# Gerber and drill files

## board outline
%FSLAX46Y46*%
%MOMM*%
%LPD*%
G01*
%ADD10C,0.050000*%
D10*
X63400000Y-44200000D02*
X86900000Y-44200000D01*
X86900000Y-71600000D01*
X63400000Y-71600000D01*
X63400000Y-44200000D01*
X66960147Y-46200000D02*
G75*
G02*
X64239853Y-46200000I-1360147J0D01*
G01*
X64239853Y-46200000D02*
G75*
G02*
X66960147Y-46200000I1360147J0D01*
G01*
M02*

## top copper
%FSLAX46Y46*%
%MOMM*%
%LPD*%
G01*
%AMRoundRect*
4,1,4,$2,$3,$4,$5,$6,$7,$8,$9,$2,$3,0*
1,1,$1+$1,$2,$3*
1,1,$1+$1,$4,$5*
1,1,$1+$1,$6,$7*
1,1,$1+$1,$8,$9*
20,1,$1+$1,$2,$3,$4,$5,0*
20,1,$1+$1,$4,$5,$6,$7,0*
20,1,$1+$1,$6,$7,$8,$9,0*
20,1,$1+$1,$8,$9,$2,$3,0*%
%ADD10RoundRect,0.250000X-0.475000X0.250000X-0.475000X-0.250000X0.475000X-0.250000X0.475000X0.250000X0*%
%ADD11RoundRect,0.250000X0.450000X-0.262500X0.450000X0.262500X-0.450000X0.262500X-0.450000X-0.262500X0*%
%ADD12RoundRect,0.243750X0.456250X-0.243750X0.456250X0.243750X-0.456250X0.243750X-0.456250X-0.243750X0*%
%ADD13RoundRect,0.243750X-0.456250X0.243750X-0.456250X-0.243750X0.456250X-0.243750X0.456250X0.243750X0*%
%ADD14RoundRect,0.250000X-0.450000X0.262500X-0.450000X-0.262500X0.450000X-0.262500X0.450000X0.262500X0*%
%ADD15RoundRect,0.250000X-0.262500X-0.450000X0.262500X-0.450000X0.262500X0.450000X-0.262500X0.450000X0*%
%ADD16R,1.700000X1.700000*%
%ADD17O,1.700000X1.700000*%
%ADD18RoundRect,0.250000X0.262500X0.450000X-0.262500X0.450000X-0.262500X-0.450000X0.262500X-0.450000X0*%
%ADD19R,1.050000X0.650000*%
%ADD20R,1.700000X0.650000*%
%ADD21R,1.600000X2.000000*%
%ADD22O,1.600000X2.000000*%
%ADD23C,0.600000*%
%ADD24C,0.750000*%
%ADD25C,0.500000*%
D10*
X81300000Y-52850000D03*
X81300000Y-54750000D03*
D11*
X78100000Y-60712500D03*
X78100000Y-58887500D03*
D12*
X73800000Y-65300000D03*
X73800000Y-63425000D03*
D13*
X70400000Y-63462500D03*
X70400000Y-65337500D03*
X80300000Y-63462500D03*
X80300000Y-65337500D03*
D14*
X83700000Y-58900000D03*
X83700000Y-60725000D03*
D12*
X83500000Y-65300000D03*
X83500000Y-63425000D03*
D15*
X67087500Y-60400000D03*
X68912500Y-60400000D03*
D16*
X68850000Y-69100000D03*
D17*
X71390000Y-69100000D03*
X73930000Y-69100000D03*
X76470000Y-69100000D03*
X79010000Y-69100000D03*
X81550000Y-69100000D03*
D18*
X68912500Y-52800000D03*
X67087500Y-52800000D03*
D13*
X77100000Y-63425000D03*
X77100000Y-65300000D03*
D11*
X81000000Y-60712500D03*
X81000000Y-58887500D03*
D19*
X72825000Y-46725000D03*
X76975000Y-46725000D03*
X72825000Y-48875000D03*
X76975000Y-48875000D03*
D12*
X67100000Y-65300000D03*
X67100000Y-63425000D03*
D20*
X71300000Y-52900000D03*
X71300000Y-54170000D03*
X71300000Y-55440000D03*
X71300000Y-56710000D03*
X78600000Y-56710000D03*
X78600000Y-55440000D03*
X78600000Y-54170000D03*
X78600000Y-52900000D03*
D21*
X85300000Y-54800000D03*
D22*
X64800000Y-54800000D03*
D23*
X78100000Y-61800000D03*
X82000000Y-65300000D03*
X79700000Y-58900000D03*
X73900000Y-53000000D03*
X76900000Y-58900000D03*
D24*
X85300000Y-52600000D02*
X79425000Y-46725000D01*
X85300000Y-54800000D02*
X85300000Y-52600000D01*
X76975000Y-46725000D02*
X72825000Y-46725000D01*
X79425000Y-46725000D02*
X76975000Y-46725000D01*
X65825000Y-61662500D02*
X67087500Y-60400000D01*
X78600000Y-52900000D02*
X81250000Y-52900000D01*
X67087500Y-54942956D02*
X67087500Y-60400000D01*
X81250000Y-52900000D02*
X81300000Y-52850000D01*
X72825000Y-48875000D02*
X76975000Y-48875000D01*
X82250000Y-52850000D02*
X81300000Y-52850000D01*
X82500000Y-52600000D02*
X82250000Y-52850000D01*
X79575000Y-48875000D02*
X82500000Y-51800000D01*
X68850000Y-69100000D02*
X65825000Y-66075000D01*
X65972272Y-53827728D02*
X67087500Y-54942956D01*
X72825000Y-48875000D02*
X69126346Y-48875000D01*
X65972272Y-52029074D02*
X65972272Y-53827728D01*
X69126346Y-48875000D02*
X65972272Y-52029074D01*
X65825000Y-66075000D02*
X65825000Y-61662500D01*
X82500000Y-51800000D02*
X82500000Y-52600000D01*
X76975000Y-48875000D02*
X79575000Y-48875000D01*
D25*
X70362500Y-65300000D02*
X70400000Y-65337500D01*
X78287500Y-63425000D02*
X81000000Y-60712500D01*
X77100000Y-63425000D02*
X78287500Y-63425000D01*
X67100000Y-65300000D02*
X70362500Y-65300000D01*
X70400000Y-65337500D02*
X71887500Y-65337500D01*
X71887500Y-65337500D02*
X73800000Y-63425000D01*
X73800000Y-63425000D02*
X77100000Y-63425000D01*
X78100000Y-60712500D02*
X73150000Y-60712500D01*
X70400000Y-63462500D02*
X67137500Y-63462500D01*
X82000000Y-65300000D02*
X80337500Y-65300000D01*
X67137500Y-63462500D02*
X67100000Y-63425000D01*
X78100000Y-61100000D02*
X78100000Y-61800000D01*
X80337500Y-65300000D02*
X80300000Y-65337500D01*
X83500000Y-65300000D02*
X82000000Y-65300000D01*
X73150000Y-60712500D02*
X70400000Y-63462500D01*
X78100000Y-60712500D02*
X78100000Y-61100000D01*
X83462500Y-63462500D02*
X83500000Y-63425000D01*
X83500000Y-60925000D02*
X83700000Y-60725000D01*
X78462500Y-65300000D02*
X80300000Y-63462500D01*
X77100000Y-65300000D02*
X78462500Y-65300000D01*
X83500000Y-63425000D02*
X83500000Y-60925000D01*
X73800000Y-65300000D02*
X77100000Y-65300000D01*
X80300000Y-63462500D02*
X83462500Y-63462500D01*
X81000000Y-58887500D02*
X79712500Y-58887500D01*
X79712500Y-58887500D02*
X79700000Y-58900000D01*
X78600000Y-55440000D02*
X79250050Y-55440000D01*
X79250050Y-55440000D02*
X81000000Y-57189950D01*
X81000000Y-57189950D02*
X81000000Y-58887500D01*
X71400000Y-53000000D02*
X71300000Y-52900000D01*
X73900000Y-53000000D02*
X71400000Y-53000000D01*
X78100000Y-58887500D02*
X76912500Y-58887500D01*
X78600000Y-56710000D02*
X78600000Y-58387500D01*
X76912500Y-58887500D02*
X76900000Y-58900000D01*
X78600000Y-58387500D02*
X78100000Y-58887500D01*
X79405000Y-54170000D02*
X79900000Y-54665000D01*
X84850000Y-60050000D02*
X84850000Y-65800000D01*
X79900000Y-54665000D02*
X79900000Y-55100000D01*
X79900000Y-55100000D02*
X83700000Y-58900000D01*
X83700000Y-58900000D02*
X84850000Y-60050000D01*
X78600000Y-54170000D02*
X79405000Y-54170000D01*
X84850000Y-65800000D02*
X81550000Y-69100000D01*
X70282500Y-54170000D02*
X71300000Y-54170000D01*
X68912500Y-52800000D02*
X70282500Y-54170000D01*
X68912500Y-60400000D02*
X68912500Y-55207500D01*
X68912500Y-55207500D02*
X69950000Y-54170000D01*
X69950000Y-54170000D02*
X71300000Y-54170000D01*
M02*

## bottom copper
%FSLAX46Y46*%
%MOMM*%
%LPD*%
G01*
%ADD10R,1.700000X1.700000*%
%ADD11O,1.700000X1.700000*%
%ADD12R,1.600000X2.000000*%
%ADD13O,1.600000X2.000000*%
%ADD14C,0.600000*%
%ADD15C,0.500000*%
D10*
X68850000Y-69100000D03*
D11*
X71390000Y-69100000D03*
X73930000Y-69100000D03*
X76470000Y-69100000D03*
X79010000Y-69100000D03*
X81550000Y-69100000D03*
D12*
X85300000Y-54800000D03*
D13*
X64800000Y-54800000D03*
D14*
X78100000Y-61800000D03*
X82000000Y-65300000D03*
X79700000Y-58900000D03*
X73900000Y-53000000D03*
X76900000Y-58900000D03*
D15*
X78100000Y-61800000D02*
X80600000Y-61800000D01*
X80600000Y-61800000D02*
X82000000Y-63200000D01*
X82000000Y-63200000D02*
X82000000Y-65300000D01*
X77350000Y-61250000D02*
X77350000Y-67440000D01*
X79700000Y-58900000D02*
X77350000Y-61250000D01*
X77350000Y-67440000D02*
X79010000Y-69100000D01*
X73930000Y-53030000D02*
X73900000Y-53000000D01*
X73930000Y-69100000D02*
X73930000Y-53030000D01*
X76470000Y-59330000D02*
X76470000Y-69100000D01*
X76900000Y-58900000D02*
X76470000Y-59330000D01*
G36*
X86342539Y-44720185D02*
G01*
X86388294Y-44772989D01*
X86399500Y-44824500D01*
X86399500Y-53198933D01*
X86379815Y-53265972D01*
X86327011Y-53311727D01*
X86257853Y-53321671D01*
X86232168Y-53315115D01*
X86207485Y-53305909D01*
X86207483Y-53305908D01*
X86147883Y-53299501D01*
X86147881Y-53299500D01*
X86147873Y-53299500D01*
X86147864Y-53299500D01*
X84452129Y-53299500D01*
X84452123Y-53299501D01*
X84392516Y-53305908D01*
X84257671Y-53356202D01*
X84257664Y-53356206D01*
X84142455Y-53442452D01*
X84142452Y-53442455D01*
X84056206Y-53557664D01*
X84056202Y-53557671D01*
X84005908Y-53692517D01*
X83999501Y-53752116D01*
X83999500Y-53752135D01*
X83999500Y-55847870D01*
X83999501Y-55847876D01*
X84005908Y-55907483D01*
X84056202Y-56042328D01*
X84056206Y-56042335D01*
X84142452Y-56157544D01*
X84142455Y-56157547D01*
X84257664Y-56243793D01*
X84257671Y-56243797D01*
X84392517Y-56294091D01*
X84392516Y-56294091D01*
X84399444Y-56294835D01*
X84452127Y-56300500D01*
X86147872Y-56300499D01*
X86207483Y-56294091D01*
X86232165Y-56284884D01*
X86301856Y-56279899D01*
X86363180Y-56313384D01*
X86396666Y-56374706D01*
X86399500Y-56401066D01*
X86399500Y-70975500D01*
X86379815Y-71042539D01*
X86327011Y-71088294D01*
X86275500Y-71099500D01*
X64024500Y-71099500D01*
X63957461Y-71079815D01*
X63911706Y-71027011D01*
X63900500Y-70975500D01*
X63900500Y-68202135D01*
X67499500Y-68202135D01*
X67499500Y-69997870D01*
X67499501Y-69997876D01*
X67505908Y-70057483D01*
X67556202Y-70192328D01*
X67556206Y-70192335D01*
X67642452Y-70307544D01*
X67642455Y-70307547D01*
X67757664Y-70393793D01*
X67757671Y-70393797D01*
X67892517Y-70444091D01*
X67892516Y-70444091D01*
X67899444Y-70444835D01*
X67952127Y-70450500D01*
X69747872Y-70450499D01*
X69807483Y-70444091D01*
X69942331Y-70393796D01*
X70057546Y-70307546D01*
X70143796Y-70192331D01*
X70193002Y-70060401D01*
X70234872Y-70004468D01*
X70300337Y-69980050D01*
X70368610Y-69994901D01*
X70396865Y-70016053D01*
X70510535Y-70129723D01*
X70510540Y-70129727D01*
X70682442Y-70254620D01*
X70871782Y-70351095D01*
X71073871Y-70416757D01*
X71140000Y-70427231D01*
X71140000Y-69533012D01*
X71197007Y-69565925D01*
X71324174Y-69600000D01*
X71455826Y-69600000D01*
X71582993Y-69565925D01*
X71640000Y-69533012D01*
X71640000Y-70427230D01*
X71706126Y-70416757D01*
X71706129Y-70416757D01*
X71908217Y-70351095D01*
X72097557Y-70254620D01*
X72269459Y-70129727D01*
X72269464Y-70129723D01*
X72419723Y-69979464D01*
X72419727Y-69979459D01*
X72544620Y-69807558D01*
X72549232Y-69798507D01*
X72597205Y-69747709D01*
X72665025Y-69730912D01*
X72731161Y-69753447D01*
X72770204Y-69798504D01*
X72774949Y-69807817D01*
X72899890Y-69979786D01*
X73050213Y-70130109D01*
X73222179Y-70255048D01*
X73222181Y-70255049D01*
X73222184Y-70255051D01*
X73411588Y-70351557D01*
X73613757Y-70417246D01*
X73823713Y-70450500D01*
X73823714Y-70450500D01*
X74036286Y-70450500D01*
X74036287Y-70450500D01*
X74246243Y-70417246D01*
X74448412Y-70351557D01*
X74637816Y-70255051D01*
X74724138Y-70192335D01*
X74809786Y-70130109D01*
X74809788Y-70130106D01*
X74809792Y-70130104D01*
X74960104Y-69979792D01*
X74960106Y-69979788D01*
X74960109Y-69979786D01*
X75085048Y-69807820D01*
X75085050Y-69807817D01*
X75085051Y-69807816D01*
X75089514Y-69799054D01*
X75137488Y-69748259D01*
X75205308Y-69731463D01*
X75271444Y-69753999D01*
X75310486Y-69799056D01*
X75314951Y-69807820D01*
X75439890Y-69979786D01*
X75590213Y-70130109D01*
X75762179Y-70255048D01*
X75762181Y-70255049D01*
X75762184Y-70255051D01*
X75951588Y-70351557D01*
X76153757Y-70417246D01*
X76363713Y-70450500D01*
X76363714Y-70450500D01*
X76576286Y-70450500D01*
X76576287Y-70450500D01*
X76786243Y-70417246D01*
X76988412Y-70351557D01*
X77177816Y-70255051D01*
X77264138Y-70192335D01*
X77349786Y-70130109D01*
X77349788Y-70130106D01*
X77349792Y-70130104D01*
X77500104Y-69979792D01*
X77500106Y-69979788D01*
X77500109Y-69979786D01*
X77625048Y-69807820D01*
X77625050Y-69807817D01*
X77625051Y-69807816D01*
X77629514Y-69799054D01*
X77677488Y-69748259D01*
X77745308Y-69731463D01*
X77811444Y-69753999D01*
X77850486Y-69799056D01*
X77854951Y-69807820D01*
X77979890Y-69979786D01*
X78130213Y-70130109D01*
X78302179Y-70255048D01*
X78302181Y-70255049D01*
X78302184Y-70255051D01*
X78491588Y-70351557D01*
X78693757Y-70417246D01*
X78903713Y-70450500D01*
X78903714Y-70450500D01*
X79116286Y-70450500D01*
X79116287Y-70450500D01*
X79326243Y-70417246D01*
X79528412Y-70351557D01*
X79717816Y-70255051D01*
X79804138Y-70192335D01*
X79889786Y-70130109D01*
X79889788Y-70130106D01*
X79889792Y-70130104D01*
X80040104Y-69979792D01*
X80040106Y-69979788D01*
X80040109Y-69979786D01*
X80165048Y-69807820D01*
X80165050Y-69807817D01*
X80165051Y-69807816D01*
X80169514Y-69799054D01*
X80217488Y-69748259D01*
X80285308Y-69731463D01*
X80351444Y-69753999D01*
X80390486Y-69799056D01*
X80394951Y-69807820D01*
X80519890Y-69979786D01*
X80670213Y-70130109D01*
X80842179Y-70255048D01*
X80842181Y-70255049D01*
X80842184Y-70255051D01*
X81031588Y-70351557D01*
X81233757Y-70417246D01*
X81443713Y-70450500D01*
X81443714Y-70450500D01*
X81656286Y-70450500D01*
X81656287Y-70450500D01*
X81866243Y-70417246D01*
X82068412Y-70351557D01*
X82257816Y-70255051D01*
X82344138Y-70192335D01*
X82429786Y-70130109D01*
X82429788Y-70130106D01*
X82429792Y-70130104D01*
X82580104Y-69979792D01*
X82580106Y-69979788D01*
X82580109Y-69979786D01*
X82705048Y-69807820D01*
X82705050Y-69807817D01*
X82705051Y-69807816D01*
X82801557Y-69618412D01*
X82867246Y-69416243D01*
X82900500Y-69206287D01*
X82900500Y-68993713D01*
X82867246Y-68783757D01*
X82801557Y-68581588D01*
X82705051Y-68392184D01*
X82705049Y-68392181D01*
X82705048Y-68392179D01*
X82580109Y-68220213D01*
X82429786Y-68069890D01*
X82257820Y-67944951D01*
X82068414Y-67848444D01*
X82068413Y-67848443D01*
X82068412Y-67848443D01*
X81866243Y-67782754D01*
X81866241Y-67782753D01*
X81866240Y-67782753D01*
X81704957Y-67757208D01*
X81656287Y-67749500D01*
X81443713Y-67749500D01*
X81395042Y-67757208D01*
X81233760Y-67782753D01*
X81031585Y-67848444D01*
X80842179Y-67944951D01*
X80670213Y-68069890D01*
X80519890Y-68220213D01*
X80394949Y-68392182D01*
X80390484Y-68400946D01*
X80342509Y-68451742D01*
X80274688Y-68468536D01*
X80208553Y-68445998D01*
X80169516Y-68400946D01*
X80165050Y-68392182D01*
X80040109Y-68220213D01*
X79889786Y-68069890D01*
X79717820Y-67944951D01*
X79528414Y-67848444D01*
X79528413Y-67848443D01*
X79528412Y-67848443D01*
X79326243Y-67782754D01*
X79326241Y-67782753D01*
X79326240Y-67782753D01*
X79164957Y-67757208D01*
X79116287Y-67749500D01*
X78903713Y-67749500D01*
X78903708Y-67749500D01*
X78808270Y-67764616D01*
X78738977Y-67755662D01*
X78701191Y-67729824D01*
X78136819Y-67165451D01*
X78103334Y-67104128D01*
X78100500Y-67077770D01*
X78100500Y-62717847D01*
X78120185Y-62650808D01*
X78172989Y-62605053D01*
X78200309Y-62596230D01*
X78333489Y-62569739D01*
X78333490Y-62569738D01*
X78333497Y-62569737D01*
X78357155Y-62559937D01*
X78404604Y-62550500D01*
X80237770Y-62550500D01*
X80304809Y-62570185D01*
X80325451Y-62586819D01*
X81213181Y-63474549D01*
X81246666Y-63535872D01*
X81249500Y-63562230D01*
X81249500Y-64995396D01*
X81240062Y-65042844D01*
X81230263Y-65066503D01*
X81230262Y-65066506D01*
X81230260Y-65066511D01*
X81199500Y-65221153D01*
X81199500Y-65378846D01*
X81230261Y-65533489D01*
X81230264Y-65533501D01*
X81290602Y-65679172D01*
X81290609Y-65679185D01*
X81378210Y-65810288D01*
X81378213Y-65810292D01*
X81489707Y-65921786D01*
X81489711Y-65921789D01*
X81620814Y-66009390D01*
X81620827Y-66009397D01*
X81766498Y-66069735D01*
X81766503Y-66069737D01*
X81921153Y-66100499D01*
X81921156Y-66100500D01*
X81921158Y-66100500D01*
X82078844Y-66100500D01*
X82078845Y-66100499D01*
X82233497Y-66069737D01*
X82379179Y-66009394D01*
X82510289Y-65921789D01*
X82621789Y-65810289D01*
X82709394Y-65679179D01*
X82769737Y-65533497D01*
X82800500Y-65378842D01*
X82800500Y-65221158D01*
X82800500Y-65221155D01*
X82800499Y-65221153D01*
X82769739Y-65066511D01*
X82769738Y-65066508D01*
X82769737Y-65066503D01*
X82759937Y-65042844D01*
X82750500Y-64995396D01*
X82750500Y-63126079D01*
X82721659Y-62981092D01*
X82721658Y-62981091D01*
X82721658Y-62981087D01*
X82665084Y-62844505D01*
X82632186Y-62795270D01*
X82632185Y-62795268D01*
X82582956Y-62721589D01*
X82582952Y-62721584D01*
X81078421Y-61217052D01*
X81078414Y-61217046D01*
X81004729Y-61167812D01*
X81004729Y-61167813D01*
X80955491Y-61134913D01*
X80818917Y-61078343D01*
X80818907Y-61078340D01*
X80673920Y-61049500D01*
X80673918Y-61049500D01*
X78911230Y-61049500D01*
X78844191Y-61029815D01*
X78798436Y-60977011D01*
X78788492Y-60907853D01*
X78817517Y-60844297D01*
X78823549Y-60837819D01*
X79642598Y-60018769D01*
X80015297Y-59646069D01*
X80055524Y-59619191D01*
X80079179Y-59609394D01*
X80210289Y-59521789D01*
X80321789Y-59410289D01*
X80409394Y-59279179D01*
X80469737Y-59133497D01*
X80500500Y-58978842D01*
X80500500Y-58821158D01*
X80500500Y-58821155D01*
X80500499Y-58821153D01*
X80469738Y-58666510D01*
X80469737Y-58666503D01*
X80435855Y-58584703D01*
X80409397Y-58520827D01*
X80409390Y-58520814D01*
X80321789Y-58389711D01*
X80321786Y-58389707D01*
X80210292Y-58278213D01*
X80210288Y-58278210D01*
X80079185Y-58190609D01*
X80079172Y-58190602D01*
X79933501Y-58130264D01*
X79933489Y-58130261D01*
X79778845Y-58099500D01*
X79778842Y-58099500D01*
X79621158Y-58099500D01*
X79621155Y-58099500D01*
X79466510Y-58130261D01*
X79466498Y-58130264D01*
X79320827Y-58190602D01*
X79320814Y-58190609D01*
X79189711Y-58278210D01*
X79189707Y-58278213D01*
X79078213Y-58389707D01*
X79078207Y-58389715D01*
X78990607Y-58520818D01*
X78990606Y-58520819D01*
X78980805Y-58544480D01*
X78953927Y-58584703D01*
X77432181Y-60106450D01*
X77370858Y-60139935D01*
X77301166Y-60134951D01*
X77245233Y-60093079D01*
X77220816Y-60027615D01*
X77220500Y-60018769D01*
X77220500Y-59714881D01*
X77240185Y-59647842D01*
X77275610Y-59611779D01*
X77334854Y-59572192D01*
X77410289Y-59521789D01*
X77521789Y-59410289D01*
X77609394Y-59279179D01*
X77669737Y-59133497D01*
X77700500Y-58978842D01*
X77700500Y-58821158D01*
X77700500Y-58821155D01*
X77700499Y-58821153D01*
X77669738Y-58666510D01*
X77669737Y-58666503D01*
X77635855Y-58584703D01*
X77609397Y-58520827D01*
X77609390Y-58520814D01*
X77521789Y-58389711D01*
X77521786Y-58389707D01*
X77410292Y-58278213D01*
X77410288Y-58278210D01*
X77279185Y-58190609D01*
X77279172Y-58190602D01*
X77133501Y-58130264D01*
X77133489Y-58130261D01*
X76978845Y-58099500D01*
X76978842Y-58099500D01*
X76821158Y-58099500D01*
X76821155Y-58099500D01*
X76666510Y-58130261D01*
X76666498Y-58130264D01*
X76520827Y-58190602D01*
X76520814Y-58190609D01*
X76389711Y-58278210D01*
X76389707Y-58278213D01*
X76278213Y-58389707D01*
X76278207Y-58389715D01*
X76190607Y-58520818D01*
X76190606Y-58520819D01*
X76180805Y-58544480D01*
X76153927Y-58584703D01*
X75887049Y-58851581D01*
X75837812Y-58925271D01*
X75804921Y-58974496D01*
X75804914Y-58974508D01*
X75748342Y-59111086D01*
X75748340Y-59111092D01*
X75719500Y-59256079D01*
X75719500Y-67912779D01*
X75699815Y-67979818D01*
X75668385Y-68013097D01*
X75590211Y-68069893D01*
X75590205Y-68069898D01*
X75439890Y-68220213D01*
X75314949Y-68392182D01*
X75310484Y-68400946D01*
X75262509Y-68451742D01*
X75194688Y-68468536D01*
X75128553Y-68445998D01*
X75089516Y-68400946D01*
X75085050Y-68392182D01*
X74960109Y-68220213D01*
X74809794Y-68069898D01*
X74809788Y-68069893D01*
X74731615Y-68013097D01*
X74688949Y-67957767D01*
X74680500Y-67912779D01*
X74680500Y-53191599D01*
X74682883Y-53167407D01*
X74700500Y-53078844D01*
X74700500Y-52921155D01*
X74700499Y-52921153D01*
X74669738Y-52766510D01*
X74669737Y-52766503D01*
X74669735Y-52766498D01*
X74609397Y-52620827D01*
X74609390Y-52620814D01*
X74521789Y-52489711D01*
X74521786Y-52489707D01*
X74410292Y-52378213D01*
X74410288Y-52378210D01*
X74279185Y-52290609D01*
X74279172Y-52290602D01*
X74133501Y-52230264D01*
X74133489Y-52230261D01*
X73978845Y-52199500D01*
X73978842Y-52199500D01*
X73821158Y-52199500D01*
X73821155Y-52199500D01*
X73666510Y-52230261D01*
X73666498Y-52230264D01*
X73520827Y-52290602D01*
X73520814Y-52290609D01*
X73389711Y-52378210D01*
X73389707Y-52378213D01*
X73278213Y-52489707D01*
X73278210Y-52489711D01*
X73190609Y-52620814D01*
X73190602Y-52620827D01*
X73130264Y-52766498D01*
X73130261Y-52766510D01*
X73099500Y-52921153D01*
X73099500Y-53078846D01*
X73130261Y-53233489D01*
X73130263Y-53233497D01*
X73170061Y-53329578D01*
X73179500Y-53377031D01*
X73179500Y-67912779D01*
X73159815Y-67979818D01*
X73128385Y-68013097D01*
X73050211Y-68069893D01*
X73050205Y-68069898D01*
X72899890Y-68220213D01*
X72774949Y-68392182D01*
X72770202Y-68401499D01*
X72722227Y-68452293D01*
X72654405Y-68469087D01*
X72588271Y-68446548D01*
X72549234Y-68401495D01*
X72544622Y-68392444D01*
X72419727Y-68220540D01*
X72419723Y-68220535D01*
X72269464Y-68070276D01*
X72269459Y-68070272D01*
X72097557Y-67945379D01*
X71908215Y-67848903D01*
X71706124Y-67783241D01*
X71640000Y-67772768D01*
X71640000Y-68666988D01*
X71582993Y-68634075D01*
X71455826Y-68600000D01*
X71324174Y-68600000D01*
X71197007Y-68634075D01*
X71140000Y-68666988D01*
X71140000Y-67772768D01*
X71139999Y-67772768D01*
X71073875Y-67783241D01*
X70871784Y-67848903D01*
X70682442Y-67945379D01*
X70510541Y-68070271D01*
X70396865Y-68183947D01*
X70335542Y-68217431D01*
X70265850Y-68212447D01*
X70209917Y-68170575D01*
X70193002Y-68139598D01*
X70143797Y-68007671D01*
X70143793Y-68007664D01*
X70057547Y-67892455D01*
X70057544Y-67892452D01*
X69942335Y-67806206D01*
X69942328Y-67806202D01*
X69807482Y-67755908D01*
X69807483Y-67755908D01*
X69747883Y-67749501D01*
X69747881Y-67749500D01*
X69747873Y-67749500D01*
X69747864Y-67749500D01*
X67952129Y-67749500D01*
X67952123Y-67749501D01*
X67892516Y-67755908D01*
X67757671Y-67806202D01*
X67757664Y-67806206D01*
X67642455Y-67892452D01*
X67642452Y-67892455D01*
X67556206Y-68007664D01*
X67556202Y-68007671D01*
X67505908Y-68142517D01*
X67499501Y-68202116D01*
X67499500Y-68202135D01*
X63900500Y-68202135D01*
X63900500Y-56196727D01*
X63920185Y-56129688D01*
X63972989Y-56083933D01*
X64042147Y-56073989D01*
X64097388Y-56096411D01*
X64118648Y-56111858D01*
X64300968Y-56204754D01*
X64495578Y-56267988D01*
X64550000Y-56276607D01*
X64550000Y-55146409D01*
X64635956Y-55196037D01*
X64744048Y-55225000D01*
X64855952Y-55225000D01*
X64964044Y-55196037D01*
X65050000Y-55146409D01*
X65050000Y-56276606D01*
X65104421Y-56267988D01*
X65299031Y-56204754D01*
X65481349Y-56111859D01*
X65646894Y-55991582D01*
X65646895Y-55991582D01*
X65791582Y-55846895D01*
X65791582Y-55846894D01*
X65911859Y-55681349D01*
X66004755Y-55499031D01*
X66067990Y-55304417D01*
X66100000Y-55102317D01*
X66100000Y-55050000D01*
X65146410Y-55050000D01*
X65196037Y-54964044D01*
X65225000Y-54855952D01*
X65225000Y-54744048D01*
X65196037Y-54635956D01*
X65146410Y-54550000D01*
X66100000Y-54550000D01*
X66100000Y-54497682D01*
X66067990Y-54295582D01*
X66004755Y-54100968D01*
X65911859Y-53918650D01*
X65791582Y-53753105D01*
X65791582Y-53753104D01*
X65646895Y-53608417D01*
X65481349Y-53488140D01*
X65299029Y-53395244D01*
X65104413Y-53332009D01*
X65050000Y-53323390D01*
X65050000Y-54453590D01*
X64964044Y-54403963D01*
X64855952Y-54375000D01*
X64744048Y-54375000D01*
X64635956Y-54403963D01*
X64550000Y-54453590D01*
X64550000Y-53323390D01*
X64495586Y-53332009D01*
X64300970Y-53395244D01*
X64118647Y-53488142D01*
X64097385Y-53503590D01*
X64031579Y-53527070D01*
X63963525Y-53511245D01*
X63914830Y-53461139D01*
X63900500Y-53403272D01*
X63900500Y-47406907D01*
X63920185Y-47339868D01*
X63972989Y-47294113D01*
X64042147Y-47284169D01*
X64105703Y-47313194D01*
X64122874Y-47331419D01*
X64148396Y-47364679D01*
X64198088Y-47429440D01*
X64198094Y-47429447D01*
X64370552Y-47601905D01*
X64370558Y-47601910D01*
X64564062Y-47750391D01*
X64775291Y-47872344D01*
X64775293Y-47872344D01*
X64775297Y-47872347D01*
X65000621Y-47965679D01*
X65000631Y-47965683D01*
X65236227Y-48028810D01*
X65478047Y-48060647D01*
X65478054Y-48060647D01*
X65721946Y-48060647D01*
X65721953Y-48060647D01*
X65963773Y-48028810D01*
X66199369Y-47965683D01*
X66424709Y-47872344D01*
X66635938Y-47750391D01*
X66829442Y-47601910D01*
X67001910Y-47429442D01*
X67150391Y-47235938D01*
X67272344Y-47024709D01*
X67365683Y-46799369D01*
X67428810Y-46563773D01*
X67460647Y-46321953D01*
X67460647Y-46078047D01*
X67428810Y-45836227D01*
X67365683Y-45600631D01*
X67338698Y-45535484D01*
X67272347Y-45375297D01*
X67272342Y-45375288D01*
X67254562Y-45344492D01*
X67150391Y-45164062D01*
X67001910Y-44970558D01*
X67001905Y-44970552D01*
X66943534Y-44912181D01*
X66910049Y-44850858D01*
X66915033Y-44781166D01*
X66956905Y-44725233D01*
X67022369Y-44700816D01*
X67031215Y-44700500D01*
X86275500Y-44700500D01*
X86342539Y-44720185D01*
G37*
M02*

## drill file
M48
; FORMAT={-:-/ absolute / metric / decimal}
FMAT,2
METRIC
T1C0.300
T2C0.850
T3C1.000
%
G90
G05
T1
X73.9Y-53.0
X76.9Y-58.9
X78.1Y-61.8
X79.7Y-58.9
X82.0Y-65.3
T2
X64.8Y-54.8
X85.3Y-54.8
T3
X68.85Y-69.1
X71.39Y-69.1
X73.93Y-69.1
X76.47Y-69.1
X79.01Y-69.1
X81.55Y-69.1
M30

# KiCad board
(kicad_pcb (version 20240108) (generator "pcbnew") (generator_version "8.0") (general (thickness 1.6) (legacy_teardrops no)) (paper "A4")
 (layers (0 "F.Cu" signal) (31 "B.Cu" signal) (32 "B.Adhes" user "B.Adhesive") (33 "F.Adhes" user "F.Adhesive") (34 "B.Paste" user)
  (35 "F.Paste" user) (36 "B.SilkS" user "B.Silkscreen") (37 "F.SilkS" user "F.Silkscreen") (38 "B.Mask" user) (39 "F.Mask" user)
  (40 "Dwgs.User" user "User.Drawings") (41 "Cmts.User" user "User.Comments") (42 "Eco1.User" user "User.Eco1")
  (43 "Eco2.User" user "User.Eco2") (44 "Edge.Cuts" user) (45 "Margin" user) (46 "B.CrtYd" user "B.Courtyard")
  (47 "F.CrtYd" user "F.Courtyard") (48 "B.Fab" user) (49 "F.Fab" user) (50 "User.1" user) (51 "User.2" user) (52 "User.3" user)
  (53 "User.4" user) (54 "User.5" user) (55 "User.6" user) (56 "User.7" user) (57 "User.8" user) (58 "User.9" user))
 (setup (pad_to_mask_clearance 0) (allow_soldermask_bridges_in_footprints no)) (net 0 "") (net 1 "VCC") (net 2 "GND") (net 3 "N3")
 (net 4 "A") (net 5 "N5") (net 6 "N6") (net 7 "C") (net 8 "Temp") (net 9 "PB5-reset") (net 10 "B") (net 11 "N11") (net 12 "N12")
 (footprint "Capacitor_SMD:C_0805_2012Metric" (layer "F.Cu") (at 81.3 53.8 -90)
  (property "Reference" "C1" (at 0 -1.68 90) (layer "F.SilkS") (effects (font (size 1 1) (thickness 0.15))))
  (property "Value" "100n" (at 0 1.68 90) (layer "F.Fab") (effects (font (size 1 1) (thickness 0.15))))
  (pad "1" smd roundrect (at -0.95 0 270) (size 1 1.45) (layers "F.Cu" "F.Paste" "F.Mask") (roundrect_rratio 0.25) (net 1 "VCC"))
  (pad "2" smd roundrect (at 0.95 0 270) (size 1 1.45) (layers "F.Cu" "F.Paste" "F.Mask") (roundrect_rratio 0.25) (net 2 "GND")))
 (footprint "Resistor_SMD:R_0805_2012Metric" (layer "F.Cu") (at 78.1 59.8 90)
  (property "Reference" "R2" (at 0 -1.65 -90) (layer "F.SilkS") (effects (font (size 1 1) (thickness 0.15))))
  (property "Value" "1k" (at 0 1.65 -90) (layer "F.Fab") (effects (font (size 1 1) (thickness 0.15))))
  (pad "1" smd roundrect (at -0.9125 0 90) (size 1.025 1.4) (layers "F.Cu" "F.Paste" "F.Mask") (roundrect_rratio 0.243902) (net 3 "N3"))
  (pad "2" smd roundrect (at 0.9125 0 90) (size 1.025 1.4) (layers "F.Cu" "F.Paste" "F.Mask") (roundrect_rratio 0.243902) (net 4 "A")))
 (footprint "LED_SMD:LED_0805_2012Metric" (layer "F.Cu") (at 73.8 64.3625 90)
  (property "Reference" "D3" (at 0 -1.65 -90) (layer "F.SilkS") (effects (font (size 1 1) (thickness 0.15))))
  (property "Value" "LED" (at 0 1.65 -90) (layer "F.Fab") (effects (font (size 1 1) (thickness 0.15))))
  (pad "1" smd roundrect (at -0.9375 0 90) (size 0.975 1.4) (layers "F.Cu" "F.Paste" "F.Mask") (roundrect_rratio 0.25) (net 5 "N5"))
  (pad "2" smd roundrect (at 0.9375 0 90) (size 0.975 1.4) (layers "F.Cu" "F.Paste" "F.Mask") (roundrect_rratio 0.25) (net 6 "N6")))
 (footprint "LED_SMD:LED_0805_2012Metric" (layer "F.Cu") (at 70.4 64.4 -90)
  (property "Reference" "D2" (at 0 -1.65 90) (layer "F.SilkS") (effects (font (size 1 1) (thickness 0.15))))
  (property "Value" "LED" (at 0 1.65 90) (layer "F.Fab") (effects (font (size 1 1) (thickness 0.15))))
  (pad "1" smd roundrect (at -0.9375 0 270) (size 0.975 1.4) (layers "F.Cu" "F.Paste" "F.Mask") (roundrect_rratio 0.25) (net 3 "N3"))
  (pad "2" smd roundrect (at 0.9375 0 270) (size 0.975 1.4) (layers "F.Cu" "F.Paste" "F.Mask") (roundrect_rratio 0.25) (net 6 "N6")))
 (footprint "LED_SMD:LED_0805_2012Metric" (layer "F.Cu") (at 80.3 64.4 -90)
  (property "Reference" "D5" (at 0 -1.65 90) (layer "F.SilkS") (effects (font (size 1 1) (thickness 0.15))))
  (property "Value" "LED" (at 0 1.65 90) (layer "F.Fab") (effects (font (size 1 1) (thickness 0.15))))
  (pad "1" smd roundrect (at -0.9375 0 270) (size 0.975 1.4) (layers "F.Cu" "F.Paste" "F.Mask") (roundrect_rratio 0.25) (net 5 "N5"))
  (pad "2" smd roundrect (at 0.9375 0 270) (size 0.975 1.4) (layers "F.Cu" "F.Paste" "F.Mask") (roundrect_rratio 0.25) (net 3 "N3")))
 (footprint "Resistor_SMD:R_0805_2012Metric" (layer "F.Cu") (at 83.7 59.8125 -90)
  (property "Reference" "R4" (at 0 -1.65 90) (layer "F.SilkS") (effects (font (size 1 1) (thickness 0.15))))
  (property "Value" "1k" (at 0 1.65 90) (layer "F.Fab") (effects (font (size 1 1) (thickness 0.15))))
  (pad "1" smd roundrect (at -0.9125 0 270) (size 1.025 1.4) (layers "F.Cu" "F.Paste" "F.Mask") (roundrect_rratio 0.243902) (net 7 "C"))
  (pad "2" smd roundrect (at 0.9125 0 270) (size 1.025 1.4) (layers "F.Cu" "F.Paste" "F.Mask") (roundrect_rratio 0.243902) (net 5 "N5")))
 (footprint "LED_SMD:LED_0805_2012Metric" (layer "F.Cu") (at 83.5 64.3625 90)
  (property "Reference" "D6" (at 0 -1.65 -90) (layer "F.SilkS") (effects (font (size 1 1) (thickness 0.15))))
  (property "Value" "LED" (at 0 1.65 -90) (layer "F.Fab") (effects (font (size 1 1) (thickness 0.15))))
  (pad "1" smd roundrect (at -0.9375 0 90) (size 0.975 1.4) (layers "F.Cu" "F.Paste" "F.Mask") (roundrect_rratio 0.25) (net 3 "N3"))
  (pad "2" smd roundrect (at 0.9375 0 90) (size 0.975 1.4) (layers "F.Cu" "F.Paste" "F.Mask") (roundrect_rratio 0.25) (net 5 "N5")))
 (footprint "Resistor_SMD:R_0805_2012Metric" (layer "F.Cu") (at 68 60.4)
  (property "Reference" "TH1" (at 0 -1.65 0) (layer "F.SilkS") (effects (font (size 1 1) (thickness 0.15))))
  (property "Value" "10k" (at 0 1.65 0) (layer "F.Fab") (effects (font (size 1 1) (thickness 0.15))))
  (pad "1" smd roundrect (at -0.9125 0) (size 1.025 1.4) (layers "F.Cu" "F.Paste" "F.Mask") (roundrect_rratio 0.243902) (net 1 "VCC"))
  (pad "2" smd roundrect (at 0.9125 0) (size 1.025 1.4) (layers "F.Cu" "F.Paste" "F.Mask") (roundrect_rratio 0.243902) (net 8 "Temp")))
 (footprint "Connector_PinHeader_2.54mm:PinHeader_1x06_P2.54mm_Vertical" (layer "F.Cu") (at 68.85 69.1 90)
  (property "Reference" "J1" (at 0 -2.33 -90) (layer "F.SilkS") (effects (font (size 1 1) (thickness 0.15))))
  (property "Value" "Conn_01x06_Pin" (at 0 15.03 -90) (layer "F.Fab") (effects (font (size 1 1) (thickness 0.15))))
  (pad "1" thru_hole rect (at 0 0 90) (size 1.7 1.7) (drill 1) (layers "*.Cu" "*.Mask") (remove_unused_layers no) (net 1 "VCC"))
  (pad "2" thru_hole oval (at 0 2.54 90) (size 1.7 1.7) (drill 1) (layers "*.Cu" "*.Mask") (remove_unused_layers no) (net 2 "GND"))
  (pad "3" thru_hole oval (at 0 5.08 90) (size 1.7 1.7) (drill 1) (layers "*.Cu" "*.Mask") (remove_unused_layers no) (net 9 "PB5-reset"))
  (pad "4" thru_hole oval (at 0 7.62 90) (size 1.7 1.7) (drill 1) (layers "*.Cu" "*.Mask") (remove_unused_layers no) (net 4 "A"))
  (pad "5" thru_hole oval (at 0 10.16 90) (size 1.7 1.7) (drill 1) (layers "*.Cu" "*.Mask") (remove_unused_layers no) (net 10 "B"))
  (pad "6" thru_hole oval (at 0 12.7 90) (size 1.7 1.7) (drill 1) (layers "*.Cu" "*.Mask") (remove_unused_layers no) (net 7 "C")))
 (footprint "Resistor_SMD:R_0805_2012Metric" (layer "F.Cu") (at 68 52.8 180)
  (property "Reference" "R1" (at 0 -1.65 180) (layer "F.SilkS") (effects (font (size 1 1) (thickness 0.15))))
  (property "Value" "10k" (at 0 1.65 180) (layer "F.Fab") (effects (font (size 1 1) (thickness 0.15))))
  (pad "1" smd roundrect (at -0.9125 0 180) (size 1.025 1.4) (layers "F.Cu" "F.Paste" "F.Mask") (roundrect_rratio 0.243902) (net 8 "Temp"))
  (pad "2" smd roundrect (at 0.9125 0 180) (size 1.025 1.4) (layers "F.Cu" "F.Paste" "F.Mask") (roundrect_rratio 0.243902) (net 2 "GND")))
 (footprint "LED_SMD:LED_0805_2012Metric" (layer "F.Cu") (at 77.1 64.3625 -90)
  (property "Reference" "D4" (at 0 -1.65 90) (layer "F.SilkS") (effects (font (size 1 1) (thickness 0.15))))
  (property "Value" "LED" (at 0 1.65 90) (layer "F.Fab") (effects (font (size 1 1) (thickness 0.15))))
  (pad "1" smd roundrect (at -0.9375 0 270) (size 0.975 1.4) (layers "F.Cu" "F.Paste" "F.Mask") (roundrect_rratio 0.25) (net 6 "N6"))
  (pad "2" smd roundrect (at 0.9375 0 270) (size 0.975 1.4) (layers "F.Cu" "F.Paste" "F.Mask") (roundrect_rratio 0.25) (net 5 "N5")))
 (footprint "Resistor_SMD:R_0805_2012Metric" (layer "F.Cu") (at 81 59.8 90)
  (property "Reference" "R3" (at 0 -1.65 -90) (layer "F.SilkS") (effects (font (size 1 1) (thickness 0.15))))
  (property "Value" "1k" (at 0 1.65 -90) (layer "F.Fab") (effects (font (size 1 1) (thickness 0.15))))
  (pad "1" smd roundrect (at -0.9125 0 90) (size 1.025 1.4) (layers "F.Cu" "F.Paste" "F.Mask") (roundrect_rratio 0.243902) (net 6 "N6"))
  (pad "2" smd roundrect (at 0.9125 0 90) (size 1.025 1.4) (layers "F.Cu" "F.Paste" "F.Mask") (roundrect_rratio 0.243902) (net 10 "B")))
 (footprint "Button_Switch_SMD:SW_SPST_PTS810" (layer "F.Cu") (at 74.9 47.8)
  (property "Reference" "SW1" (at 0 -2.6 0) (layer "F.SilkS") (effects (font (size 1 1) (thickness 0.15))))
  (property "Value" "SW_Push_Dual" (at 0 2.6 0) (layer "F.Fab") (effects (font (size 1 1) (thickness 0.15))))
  (pad "1" smd rect (at -2.075 -1.075) (size 1.05 0.65) (layers "F.Cu" "F.Paste" "F.Mask") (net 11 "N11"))
  (pad "1" smd rect (at 2.075 -1.075) (size 1.05 0.65) (layers "F.Cu" "F.Paste" "F.Mask") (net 11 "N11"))
  (pad "2" smd rect (at -2.075 1.075) (size 1.05 0.65) (layers "F.Cu" "F.Paste" "F.Mask") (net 1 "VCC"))
  (pad "2" smd rect (at 2.075 1.075) (size 1.05 0.65) (layers "F.Cu" "F.Paste" "F.Mask") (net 1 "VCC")))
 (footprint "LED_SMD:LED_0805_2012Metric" (layer "F.Cu") (at 67.1 64.3625 90)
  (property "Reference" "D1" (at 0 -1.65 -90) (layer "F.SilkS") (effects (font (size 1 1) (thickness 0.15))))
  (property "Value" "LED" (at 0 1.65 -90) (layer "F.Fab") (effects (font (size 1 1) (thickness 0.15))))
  (pad "1" smd roundrect (at -0.9375 0 90) (size 0.975 1.4) (layers "F.Cu" "F.Paste" "F.Mask") (roundrect_rratio 0.25) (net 6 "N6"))
  (pad "2" smd roundrect (at 0.9375 0 90) (size 0.975 1.4) (layers "F.Cu" "F.Paste" "F.Mask") (roundrect_rratio 0.25) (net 3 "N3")))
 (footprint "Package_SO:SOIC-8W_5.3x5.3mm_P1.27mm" (layer "F.Cu") (at 74.95 54.805)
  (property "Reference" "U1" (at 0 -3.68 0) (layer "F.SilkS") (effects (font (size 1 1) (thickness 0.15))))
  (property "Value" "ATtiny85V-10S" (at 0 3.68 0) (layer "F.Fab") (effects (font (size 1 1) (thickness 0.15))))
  (pad "1" smd rect (at -3.65 -1.905) (size 1.7 0.65) (layers "F.Cu" "F.Paste" "F.Mask") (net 9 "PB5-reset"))
  (pad "2" smd rect (at -3.65 -0.635) (size 1.7 0.65) (layers "F.Cu" "F.Paste" "F.Mask") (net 8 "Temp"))
  (pad "3" smd rect (at -3.65 0.635) (size 1.7 0.65) (layers "F.Cu" "F.Paste" "F.Mask") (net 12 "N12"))
  (pad "4" smd rect (at -3.65 1.905) (size 1.7 0.65) (layers "F.Cu" "F.Paste" "F.Mask") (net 2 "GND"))
  (pad "5" smd rect (at 3.65 1.905) (size 1.7 0.65) (layers "F.Cu" "F.Paste" "F.Mask") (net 4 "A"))
  (pad "6" smd rect (at 3.65 0.635) (size 1.7 0.65) (layers "F.Cu" "F.Paste" "F.Mask") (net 10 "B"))
  (pad "7" smd rect (at 3.65 -0.635) (size 1.7 0.65) (layers "F.Cu" "F.Paste" "F.Mask") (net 7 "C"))
  (pad "8" smd rect (at 3.65 -1.905) (size 1.7 0.65) (layers "F.Cu" "F.Paste" "F.Mask") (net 1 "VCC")))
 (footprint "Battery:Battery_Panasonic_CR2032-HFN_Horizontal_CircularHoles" (layer "B.Cu") (at 85.3 54.8 180)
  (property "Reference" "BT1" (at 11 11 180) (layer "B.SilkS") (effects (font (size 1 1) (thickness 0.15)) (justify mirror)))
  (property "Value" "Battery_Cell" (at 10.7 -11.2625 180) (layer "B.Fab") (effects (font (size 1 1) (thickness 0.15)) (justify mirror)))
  (pad "1" thru_hole rect (at 0 0 180) (size 1.6 2) (drill 0.85) (layers "*.Cu" "*.Mask") (remove_unused_layers no) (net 11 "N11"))
  (pad "2" thru_hole oval (at 20.5 0 180) (size 1.6 2) (drill 0.85) (layers "*.Cu" "*.Mask") (remove_unused_layers no) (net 2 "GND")))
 (gr_rect (start 63.4 44.2) (end 86.9 71.6) (stroke (width 0.05) (type default)) (fill none) (layer "Edge.Cuts"))
 (gr_circle (center 65.6 46.2) (end 66.4 47.3) (stroke (width 0.05) (type default)) (fill none) (layer "Edge.Cuts"))
 (segment (start 85.3 52.6) (end 79.425 46.725) (width 0.75) (layer "F.Cu") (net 11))
 (segment (start 85.3 54.8) (end 85.3 52.6) (width 0.75) (layer "F.Cu") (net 11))
 (segment (start 76.975 46.725) (end 72.825 46.725) (width 0.75) (layer "F.Cu") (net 11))
 (segment (start 79.425 46.725) (end 76.975 46.725) (width 0.75) (layer "F.Cu") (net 11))
 (segment (start 65.825 61.6625) (end 67.0875 60.4) (width 0.75) (layer "F.Cu") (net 1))
 (segment (start 78.6 52.9) (end 81.25 52.9) (width 0.75) (layer "F.Cu") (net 1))
 (segment (start 67.0875 54.942956) (end 67.0875 60.4) (width 0.75) (layer "F.Cu") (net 1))
 (segment (start 81.25 52.9) (end 81.3 52.85) (width 0.75) (layer "F.Cu") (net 1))
 (segment (start 72.825 48.875) (end 76.975 48.875) (width 0.75) (layer "F.Cu") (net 1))
 (segment (start 82.25 52.85) (end 81.3 52.85) (width 0.75) (layer "F.Cu") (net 1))
 (segment (start 82.5 52.6) (end 82.25 52.85) (width 0.75) (layer "F.Cu") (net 1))
 (segment (start 79.575 48.875) (end 82.5 51.8) (width 0.75) (layer "F.Cu") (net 1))
 (segment (start 68.85 69.1) (end 65.825 66.075) (width 0.75) (layer "F.Cu") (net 1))
 (segment (start 65.972272 53.827728) (end 67.0875 54.942956) (width 0.75) (layer "F.Cu") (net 1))
 (segment (start 72.825 48.875) (end 69.126346 48.875) (width 0.75) (layer "F.Cu") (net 1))
 (segment (start 65.972272 52.029074) (end 65.972272 53.827728) (width 0.75) (layer "F.Cu") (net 1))
 (segment (start 69.126346 48.875) (end 65.972272 52.029074) (width 0.75) (layer "F.Cu") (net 1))
 (segment (start 65.825 66.075) (end 65.825 61.6625) (width 0.75) (layer "F.Cu") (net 1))
 (segment (start 82.5 51.8) (end 82.5 52.6) (width 0.75) (layer "F.Cu") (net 1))
 (segment (start 76.975 48.875) (end 79.575 48.875) (width 0.75) (layer "F.Cu") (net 1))
 (segment (start 70.3625 65.3) (end 70.4 65.3375) (width 0.5) (layer "F.Cu") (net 6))
 (segment (start 78.2875 63.425) (end 81 60.7125) (width 0.5) (layer "F.Cu") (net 6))
 (segment (start 77.1 63.425) (end 78.2875 63.425) (width 0.5) (layer "F.Cu") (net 6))
 (segment (start 67.1 65.3) (end 70.3625 65.3) (width 0.5) (layer "F.Cu") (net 6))
 (segment (start 70.4 65.3375) (end 71.8875 65.3375) (width 0.5) (layer "F.Cu") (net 6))
 (segment (start 71.8875 65.3375) (end 73.8 63.425) (width 0.5) (layer "F.Cu") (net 6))
 (segment (start 73.8 63.425) (end 77.1 63.425) (width 0.5) (layer "F.Cu") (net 6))
 (segment (start 78.1 60.7125) (end 73.15 60.7125) (width 0.5) (layer "F.Cu") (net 3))
 (segment (start 70.4 63.4625) (end 67.1375 63.4625) (width 0.5) (layer "F.Cu") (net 3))
 (segment (start 82 65.3) (end 80.3375 65.3) (width 0.5) (layer "F.Cu") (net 3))
 (segment (start 67.1375 63.4625) (end 67.1 63.425) (width 0.5) (layer "F.Cu") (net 3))
 (segment (start 78.1 61.1) (end 78.1 61.8) (width 0.5) (layer "F.Cu") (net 3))
 (segment (start 80.3375 65.3) (end 80.3 65.3375) (width 0.5) (layer "F.Cu") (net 3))
 (segment (start 83.5 65.3) (end 82 65.3) (width 0.5) (layer "F.Cu") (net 3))
 (segment (start 73.15 60.7125) (end 70.4 63.4625) (width 0.5) (layer "F.Cu") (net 3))
 (segment (start 78.1 60.7125) (end 78.1 61.1) (width 0.5) (layer "F.Cu") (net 3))
 (via (at 78.1 61.8) (size 0.6) (drill 0.3) (layers "F.Cu" "B.Cu") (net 3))
 (via (at 82 65.3) (size 0.6) (drill 0.3) (layers "F.Cu" "B.Cu") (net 3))
 (segment (start 78.1 61.8) (end 80.6 61.8) (width 0.5) (layer "B.Cu") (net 3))
 (segment (start 80.6 61.8) (end 82 63.2) (width 0.5) (layer "B.Cu") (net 3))
 (segment (start 82 63.2) (end 82 65.3) (width 0.5) (layer "B.Cu") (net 3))
 (segment (start 83.4625 63.4625) (end 83.5 63.425) (width 0.5) (layer "F.Cu") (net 5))
 (segment (start 83.5 60.925) (end 83.7 60.725) (width 0.5) (layer "F.Cu") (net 5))
 (segment (start 78.4625 65.3) (end 80.3 63.4625) (width 0.5) (layer "F.Cu") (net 5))
 (segment (start 77.1 65.3) (end 78.4625 65.3) (width 0.5) (layer "F.Cu") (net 5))
 (segment (start 83.5 63.425) (end 83.5 60.925) (width 0.5) (layer "F.Cu") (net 5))
 (segment (start 73.8 65.3) (end 77.1 65.3) (width 0.5) (layer "F.Cu") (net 5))
 (segment (start 80.3 63.4625) (end 83.4625 63.4625) (width 0.5) (layer "F.Cu") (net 5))
 (segment (start 81 58.8875) (end 79.7125 58.8875) (width 0.5) (layer "F.Cu") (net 10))
 (segment (start 79.7125 58.8875) (end 79.7 58.9) (width 0.5) (layer "F.Cu") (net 10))
 (segment (start 78.6 55.44) (end 79.25005 55.44) (width 0.5) (layer "F.Cu") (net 10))
 (segment (start 79.25005 55.44) (end 81 57.18995) (width 0.5) (layer "F.Cu") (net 10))
 (segment (start 81 57.18995) (end 81 58.8875) (width 0.5) (layer "F.Cu") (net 10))
 (via (at 79.7 58.9) (size 0.6) (drill 0.3) (layers "F.Cu" "B.Cu") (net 10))
 (segment (start 77.35 61.25) (end 77.35 67.44) (width 0.5) (layer "B.Cu") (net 10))
 (segment (start 79.7 58.9) (end 77.35 61.25) (width 0.5) (layer "B.Cu") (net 10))
 (segment (start 77.35 67.44) (end 79.01 69.1) (width 0.5) (layer "B.Cu") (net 10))
 (segment (start 71.4 53) (end 71.3 52.9) (width 0.5) (layer "F.Cu") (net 9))
 (segment (start 73.9 53) (end 71.4 53) (width 0.5) (layer "F.Cu") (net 9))
 (via (at 73.9 53) (size 0.6) (drill 0.3) (layers "F.Cu" "B.Cu") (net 9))
 (segment (start 73.93 53.03) (end 73.9 53) (width 0.5) (layer "B.Cu") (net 9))
 (segment (start 73.93 69.1) (end 73.93 53.03) (width 0.5) (layer "B.Cu") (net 9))
 (segment (start 78.1 58.8875) (end 76.9125 58.8875) (width 0.5) (layer "F.Cu") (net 4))
 (segment (start 78.6 56.71) (end 78.6 58.3875) (width 0.5) (layer "F.Cu") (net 4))
 (segment (start 76.9125 58.8875) (end 76.9 58.9) (width 0.5) (layer "F.Cu") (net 4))
 (segment (start 78.6 58.3875) (end 78.1 58.8875) (width 0.5) (layer "F.Cu") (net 4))
 (via (at 76.9 58.9) (size 0.6) (drill 0.3) (layers "F.Cu" "B.Cu") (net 4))
 (segment (start 76.47 59.33) (end 76.47 69.1) (width 0.5) (layer "B.Cu") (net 4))
 (segment (start 76.9 58.9) (end 76.47 59.33) (width 0.5) (layer "B.Cu") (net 4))
 (segment (start 79.405 54.17) (end 79.9 54.665) (width 0.5) (layer "F.Cu") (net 7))
 (segment (start 84.85 60.05) (end 84.85 65.8) (width 0.5) (layer "F.Cu") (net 7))
 (segment (start 79.9 54.665) (end 79.9 55.1) (width 0.5) (layer "F.Cu") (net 7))
 (segment (start 79.9 55.1) (end 83.7 58.9) (width 0.5) (layer "F.Cu") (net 7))
 (segment (start 83.7 58.9) (end 84.85 60.05) (width 0.5) (layer "F.Cu") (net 7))
 (segment (start 78.6 54.17) (end 79.405 54.17) (width 0.5) (layer "F.Cu") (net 7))
 (segment (start 84.85 65.8) (end 81.55 69.1) (width 0.5) (layer "F.Cu") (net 7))
 (segment (start 70.2825 54.17) (end 71.3 54.17) (width 0.5) (layer "F.Cu") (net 8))
 (segment (start 68.9125 52.8) (end 70.2825 54.17) (width 0.5) (layer "F.Cu") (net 8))
 (segment (start 68.9125 60.4) (end 68.9125 55.2075) (width 0.5) (layer "F.Cu") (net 8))
 (segment (start 68.9125 55.2075) (end 69.95 54.17) (width 0.5) (layer "F.Cu") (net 8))
 (segment (start 69.95 54.17) (end 71.3 54.17) (width 0.5) (layer "F.Cu") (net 8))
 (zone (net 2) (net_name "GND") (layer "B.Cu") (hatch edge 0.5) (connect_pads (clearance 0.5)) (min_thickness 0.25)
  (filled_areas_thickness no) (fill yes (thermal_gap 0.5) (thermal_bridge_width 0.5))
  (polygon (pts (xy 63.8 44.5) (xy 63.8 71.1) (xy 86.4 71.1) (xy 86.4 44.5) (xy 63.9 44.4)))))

